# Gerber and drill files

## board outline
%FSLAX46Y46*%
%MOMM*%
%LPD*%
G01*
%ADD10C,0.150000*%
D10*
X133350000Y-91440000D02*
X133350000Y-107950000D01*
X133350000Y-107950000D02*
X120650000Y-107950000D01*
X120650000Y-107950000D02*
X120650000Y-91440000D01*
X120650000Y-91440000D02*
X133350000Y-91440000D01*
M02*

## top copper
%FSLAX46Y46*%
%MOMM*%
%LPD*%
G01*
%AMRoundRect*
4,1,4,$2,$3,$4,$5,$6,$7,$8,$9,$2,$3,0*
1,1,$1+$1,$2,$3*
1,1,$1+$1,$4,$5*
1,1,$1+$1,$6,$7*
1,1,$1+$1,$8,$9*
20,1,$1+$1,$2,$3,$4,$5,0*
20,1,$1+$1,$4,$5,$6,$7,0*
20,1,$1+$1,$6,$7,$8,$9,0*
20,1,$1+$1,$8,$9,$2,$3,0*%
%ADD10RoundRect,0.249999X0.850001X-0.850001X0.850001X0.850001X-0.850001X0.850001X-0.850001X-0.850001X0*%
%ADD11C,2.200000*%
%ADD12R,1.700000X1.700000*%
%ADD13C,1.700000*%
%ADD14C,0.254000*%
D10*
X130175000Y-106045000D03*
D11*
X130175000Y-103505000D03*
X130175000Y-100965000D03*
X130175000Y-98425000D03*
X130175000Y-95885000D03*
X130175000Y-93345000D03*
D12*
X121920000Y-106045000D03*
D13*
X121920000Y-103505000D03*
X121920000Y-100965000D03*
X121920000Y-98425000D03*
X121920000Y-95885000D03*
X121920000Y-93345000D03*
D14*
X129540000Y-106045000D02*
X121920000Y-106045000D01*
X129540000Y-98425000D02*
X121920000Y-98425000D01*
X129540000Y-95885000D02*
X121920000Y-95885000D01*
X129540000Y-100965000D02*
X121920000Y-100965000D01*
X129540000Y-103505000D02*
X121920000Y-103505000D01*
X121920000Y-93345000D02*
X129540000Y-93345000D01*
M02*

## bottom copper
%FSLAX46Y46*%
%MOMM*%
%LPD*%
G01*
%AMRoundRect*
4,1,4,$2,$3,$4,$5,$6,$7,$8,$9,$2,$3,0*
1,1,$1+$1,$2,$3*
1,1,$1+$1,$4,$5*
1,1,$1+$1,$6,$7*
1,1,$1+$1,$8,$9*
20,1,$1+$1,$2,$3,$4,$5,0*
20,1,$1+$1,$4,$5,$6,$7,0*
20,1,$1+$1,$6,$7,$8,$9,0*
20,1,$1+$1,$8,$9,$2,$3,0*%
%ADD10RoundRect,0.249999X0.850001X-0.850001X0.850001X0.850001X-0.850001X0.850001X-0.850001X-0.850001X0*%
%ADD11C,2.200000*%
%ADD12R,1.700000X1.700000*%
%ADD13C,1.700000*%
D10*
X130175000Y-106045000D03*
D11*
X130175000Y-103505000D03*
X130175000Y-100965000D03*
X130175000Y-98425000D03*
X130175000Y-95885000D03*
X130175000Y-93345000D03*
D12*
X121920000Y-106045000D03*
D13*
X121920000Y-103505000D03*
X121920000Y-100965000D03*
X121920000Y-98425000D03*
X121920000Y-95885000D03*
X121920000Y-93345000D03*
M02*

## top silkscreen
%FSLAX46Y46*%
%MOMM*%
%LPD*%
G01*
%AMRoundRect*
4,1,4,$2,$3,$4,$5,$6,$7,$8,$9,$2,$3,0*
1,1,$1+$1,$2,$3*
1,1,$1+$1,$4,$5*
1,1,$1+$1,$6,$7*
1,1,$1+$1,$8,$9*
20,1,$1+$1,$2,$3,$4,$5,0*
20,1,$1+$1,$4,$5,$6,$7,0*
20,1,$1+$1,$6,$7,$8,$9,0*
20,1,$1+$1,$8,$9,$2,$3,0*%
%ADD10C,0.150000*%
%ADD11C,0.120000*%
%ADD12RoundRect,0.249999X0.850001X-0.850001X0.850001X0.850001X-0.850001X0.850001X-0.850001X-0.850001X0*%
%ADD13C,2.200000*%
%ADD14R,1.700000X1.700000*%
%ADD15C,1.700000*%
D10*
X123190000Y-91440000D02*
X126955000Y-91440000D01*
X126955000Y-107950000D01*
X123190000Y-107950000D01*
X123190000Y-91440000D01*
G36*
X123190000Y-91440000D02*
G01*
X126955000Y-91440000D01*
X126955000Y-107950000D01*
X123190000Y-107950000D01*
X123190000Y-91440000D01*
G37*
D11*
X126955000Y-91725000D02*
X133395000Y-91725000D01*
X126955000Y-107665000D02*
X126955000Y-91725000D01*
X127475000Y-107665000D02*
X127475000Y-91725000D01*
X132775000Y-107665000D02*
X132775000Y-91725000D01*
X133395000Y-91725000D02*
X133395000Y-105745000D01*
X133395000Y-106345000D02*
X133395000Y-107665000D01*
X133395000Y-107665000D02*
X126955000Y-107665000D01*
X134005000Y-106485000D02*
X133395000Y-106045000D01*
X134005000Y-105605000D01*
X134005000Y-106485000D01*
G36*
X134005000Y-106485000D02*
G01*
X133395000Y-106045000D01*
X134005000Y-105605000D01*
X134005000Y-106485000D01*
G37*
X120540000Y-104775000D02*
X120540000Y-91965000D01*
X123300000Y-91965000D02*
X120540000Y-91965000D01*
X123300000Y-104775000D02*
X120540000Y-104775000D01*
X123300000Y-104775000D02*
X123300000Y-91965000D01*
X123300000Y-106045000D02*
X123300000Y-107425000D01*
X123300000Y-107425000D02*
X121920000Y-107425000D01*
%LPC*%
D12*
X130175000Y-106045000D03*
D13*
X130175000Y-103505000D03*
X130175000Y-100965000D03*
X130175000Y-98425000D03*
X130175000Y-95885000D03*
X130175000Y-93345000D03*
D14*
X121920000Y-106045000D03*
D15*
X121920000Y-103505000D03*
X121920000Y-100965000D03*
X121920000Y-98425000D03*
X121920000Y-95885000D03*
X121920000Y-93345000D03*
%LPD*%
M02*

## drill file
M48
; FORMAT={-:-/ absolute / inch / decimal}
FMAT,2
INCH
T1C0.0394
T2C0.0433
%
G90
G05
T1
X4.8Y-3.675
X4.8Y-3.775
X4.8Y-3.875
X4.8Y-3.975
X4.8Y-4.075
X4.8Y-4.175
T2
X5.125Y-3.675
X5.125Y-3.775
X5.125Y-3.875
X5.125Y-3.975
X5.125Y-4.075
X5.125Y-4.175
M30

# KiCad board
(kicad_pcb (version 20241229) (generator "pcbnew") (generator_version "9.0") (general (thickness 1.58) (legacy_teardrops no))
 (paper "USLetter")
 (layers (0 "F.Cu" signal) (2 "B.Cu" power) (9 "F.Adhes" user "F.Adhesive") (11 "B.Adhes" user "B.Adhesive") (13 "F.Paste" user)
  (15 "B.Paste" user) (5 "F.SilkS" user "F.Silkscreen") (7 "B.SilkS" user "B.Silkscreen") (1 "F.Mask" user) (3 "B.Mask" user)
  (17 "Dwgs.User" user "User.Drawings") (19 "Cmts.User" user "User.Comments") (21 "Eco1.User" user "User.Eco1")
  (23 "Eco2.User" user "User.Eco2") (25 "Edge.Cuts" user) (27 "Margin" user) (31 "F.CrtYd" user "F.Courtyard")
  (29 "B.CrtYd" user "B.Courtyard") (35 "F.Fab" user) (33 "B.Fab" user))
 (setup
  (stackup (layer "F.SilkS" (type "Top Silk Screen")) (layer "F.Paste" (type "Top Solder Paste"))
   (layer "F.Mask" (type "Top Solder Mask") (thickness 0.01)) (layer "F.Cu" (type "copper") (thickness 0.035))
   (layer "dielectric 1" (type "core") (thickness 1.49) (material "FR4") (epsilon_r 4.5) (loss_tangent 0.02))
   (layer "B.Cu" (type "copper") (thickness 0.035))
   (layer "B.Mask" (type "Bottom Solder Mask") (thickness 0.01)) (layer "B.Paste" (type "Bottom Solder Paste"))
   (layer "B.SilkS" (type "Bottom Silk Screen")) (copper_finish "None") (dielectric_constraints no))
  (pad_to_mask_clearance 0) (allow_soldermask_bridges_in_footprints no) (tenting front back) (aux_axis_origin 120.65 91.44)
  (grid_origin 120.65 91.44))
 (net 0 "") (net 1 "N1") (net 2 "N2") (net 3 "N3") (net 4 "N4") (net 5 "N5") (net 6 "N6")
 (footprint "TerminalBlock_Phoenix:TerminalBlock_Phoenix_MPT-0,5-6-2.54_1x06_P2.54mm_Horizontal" (layer "F.Cu") (at 130.175 106.045 90)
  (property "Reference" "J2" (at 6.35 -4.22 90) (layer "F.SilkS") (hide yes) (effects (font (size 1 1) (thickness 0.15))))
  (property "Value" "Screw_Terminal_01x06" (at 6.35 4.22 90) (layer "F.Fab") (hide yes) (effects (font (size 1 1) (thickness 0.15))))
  (fp_line (start 14.32 -3.22) (end 14.32 3.22) (stroke (width 0.12) (type solid)) (layer "F.SilkS"))
  (fp_line (start -1.62 -3.22) (end 14.32 -3.22) (stroke (width 0.12) (type solid)) (layer "F.SilkS"))
  (fp_line (start -1.62 -2.7) (end 14.32 -2.7) (stroke (width 0.12) (type solid)) (layer "F.SilkS"))
  (fp_line (start -1.62 2.6) (end 14.32 2.6) (stroke (width 0.12) (type solid)) (layer "F.SilkS"))
  (fp_line (start 14.32 3.22) (end 0.3 3.22) (stroke (width 0.12) (type solid)) (layer "F.SilkS"))
  (fp_line (start -0.3 3.22) (end -1.62 3.22) (stroke (width 0.12) (type solid)) (layer "F.SilkS"))
  (fp_line (start -1.62 3.22) (end -1.62 -3.22) (stroke (width 0.12) (type solid)) (layer "F.SilkS"))
  (fp_poly (pts (xy 0 3.22) (xy 0.44 3.83) (xy -0.44 3.83)) (stroke (width 0.12) (type solid)) (fill yes) (layer "F.SilkS"))
  (pad "1" thru_hole roundrect (at 0 0 90) (size 2.2 2.2) (drill 1.1) (layers "*.Cu" "*.Mask") (remove_unused_layers no)
   (roundrect_rratio 0.113636) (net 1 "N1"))
  (pad "2" thru_hole circle (at 2.54 0 90) (size 2.2 2.2) (drill 1.1) (layers "*.Cu" "*.Mask") (remove_unused_layers no) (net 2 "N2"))
  (pad "3" thru_hole circle (at 5.08 0 90) (size 2.2 2.2) (drill 1.1) (layers "*.Cu" "*.Mask") (remove_unused_layers no) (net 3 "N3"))
  (pad "4" thru_hole circle (at 7.62 0 90) (size 2.2 2.2) (drill 1.1) (layers "*.Cu" "*.Mask") (remove_unused_layers no) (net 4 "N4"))
  (pad "5" thru_hole circle (at 10.16 0 90) (size 2.2 2.2) (drill 1.1) (layers "*.Cu" "*.Mask") (remove_unused_layers no) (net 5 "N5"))
  (pad "6" thru_hole circle (at 12.7 0 90) (size 2.2 2.2) (drill 1.1) (layers "*.Cu" "*.Mask") (remove_unused_layers no) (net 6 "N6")))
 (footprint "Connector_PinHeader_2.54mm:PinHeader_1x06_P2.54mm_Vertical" (layer "F.Cu") (at 121.92 106.045 180)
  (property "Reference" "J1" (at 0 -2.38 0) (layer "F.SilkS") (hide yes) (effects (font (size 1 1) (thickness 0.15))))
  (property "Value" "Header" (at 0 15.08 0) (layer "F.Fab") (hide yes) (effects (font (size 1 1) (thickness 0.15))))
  (fp_line (start 1.38 1.27) (end 1.38 14.08) (stroke (width 0.12) (type solid)) (layer "F.SilkS"))
  (fp_line (start -1.38 14.08) (end 1.38 14.08) (stroke (width 0.12) (type solid)) (layer "F.SilkS"))
  (fp_line (start -1.38 1.27) (end 1.38 1.27) (stroke (width 0.12) (type solid)) (layer "F.SilkS"))
  (fp_line (start -1.38 1.27) (end -1.38 14.08) (stroke (width 0.12) (type solid)) (layer "F.SilkS"))
  (fp_line (start -1.38 0) (end -1.38 -1.38) (stroke (width 0.12) (type solid)) (layer "F.SilkS"))
  (fp_line (start -1.38 -1.38) (end 0 -1.38) (stroke (width 0.12) (type solid)) (layer "F.SilkS"))
  (pad "1" thru_hole rect (at 0 0 180) (size 1.7 1.7) (drill 1) (layers "*.Cu" "*.Mask") (remove_unused_layers no) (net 1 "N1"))
  (pad "2" thru_hole circle (at 0 2.54 180) (size 1.7 1.7) (drill 1) (layers "*.Cu" "*.Mask") (remove_unused_layers no) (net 2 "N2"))
  (pad "3" thru_hole circle (at 0 5.08 180) (size 1.7 1.7) (drill 1) (layers "*.Cu" "*.Mask") (remove_unused_layers no) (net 3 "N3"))
  (pad "4" thru_hole circle (at 0 7.62 180) (size 1.7 1.7) (drill 1) (layers "*.Cu" "*.Mask") (remove_unused_layers no) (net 4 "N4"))
  (pad "5" thru_hole circle (at 0 10.16 180) (size 1.7 1.7) (drill 1) (layers "*.Cu" "*.Mask") (remove_unused_layers no) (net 5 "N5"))
  (pad "6" thru_hole circle (at 0 12.7 180) (size 1.7 1.7) (drill 1) (layers "*.Cu" "*.Mask") (remove_unused_layers no) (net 6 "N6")))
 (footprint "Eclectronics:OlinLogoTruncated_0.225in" (layer "B.Cu") (at 125.857 97.663 90)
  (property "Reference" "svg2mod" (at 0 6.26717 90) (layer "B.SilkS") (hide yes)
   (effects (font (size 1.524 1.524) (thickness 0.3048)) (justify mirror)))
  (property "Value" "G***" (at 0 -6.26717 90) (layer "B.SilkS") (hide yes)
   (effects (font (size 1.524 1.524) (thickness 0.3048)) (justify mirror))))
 (gr_rect (start 123.19 91.44) (end 126.955 107.95) (stroke (width 0.15) (type solid)) (fill yes) (layer "F.SilkS"))
 (gr_line (start 133.35 91.44) (end 133.35 107.95) (stroke (width 0.15) (type default)) (layer "Edge.Cuts"))
 (gr_line (start 133.35 107.95) (end 120.65 107.95) (stroke (width 0.15) (type default)) (layer "Edge.Cuts"))
 (gr_line (start 120.65 107.95) (end 120.65 91.44) (stroke (width 0.15) (type default)) (layer "Edge.Cuts"))
 (gr_line (start 120.65 91.44) (end 133.35 91.44) (stroke (width 0.15) (type default)) (layer "Edge.Cuts"))
 (segment (start 129.54 106.045) (end 121.92 106.045) (width 0.254) (layer "F.Cu") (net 1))
 (segment (start 129.54 98.425) (end 121.92 98.425) (width 0.254) (layer "F.Cu") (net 4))
 (segment (start 129.54 95.885) (end 121.92 95.885) (width 0.254) (layer "F.Cu") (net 5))
 (segment (start 129.54 100.965) (end 121.92 100.965) (width 0.254) (layer "F.Cu") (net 3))
 (segment (start 129.54 103.505) (end 121.92 103.505) (width 0.254) (layer "F.Cu") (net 2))
 (segment (start 121.92 93.345) (end 129.54 93.345) (width 0.254) (layer "F.Cu") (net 6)))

